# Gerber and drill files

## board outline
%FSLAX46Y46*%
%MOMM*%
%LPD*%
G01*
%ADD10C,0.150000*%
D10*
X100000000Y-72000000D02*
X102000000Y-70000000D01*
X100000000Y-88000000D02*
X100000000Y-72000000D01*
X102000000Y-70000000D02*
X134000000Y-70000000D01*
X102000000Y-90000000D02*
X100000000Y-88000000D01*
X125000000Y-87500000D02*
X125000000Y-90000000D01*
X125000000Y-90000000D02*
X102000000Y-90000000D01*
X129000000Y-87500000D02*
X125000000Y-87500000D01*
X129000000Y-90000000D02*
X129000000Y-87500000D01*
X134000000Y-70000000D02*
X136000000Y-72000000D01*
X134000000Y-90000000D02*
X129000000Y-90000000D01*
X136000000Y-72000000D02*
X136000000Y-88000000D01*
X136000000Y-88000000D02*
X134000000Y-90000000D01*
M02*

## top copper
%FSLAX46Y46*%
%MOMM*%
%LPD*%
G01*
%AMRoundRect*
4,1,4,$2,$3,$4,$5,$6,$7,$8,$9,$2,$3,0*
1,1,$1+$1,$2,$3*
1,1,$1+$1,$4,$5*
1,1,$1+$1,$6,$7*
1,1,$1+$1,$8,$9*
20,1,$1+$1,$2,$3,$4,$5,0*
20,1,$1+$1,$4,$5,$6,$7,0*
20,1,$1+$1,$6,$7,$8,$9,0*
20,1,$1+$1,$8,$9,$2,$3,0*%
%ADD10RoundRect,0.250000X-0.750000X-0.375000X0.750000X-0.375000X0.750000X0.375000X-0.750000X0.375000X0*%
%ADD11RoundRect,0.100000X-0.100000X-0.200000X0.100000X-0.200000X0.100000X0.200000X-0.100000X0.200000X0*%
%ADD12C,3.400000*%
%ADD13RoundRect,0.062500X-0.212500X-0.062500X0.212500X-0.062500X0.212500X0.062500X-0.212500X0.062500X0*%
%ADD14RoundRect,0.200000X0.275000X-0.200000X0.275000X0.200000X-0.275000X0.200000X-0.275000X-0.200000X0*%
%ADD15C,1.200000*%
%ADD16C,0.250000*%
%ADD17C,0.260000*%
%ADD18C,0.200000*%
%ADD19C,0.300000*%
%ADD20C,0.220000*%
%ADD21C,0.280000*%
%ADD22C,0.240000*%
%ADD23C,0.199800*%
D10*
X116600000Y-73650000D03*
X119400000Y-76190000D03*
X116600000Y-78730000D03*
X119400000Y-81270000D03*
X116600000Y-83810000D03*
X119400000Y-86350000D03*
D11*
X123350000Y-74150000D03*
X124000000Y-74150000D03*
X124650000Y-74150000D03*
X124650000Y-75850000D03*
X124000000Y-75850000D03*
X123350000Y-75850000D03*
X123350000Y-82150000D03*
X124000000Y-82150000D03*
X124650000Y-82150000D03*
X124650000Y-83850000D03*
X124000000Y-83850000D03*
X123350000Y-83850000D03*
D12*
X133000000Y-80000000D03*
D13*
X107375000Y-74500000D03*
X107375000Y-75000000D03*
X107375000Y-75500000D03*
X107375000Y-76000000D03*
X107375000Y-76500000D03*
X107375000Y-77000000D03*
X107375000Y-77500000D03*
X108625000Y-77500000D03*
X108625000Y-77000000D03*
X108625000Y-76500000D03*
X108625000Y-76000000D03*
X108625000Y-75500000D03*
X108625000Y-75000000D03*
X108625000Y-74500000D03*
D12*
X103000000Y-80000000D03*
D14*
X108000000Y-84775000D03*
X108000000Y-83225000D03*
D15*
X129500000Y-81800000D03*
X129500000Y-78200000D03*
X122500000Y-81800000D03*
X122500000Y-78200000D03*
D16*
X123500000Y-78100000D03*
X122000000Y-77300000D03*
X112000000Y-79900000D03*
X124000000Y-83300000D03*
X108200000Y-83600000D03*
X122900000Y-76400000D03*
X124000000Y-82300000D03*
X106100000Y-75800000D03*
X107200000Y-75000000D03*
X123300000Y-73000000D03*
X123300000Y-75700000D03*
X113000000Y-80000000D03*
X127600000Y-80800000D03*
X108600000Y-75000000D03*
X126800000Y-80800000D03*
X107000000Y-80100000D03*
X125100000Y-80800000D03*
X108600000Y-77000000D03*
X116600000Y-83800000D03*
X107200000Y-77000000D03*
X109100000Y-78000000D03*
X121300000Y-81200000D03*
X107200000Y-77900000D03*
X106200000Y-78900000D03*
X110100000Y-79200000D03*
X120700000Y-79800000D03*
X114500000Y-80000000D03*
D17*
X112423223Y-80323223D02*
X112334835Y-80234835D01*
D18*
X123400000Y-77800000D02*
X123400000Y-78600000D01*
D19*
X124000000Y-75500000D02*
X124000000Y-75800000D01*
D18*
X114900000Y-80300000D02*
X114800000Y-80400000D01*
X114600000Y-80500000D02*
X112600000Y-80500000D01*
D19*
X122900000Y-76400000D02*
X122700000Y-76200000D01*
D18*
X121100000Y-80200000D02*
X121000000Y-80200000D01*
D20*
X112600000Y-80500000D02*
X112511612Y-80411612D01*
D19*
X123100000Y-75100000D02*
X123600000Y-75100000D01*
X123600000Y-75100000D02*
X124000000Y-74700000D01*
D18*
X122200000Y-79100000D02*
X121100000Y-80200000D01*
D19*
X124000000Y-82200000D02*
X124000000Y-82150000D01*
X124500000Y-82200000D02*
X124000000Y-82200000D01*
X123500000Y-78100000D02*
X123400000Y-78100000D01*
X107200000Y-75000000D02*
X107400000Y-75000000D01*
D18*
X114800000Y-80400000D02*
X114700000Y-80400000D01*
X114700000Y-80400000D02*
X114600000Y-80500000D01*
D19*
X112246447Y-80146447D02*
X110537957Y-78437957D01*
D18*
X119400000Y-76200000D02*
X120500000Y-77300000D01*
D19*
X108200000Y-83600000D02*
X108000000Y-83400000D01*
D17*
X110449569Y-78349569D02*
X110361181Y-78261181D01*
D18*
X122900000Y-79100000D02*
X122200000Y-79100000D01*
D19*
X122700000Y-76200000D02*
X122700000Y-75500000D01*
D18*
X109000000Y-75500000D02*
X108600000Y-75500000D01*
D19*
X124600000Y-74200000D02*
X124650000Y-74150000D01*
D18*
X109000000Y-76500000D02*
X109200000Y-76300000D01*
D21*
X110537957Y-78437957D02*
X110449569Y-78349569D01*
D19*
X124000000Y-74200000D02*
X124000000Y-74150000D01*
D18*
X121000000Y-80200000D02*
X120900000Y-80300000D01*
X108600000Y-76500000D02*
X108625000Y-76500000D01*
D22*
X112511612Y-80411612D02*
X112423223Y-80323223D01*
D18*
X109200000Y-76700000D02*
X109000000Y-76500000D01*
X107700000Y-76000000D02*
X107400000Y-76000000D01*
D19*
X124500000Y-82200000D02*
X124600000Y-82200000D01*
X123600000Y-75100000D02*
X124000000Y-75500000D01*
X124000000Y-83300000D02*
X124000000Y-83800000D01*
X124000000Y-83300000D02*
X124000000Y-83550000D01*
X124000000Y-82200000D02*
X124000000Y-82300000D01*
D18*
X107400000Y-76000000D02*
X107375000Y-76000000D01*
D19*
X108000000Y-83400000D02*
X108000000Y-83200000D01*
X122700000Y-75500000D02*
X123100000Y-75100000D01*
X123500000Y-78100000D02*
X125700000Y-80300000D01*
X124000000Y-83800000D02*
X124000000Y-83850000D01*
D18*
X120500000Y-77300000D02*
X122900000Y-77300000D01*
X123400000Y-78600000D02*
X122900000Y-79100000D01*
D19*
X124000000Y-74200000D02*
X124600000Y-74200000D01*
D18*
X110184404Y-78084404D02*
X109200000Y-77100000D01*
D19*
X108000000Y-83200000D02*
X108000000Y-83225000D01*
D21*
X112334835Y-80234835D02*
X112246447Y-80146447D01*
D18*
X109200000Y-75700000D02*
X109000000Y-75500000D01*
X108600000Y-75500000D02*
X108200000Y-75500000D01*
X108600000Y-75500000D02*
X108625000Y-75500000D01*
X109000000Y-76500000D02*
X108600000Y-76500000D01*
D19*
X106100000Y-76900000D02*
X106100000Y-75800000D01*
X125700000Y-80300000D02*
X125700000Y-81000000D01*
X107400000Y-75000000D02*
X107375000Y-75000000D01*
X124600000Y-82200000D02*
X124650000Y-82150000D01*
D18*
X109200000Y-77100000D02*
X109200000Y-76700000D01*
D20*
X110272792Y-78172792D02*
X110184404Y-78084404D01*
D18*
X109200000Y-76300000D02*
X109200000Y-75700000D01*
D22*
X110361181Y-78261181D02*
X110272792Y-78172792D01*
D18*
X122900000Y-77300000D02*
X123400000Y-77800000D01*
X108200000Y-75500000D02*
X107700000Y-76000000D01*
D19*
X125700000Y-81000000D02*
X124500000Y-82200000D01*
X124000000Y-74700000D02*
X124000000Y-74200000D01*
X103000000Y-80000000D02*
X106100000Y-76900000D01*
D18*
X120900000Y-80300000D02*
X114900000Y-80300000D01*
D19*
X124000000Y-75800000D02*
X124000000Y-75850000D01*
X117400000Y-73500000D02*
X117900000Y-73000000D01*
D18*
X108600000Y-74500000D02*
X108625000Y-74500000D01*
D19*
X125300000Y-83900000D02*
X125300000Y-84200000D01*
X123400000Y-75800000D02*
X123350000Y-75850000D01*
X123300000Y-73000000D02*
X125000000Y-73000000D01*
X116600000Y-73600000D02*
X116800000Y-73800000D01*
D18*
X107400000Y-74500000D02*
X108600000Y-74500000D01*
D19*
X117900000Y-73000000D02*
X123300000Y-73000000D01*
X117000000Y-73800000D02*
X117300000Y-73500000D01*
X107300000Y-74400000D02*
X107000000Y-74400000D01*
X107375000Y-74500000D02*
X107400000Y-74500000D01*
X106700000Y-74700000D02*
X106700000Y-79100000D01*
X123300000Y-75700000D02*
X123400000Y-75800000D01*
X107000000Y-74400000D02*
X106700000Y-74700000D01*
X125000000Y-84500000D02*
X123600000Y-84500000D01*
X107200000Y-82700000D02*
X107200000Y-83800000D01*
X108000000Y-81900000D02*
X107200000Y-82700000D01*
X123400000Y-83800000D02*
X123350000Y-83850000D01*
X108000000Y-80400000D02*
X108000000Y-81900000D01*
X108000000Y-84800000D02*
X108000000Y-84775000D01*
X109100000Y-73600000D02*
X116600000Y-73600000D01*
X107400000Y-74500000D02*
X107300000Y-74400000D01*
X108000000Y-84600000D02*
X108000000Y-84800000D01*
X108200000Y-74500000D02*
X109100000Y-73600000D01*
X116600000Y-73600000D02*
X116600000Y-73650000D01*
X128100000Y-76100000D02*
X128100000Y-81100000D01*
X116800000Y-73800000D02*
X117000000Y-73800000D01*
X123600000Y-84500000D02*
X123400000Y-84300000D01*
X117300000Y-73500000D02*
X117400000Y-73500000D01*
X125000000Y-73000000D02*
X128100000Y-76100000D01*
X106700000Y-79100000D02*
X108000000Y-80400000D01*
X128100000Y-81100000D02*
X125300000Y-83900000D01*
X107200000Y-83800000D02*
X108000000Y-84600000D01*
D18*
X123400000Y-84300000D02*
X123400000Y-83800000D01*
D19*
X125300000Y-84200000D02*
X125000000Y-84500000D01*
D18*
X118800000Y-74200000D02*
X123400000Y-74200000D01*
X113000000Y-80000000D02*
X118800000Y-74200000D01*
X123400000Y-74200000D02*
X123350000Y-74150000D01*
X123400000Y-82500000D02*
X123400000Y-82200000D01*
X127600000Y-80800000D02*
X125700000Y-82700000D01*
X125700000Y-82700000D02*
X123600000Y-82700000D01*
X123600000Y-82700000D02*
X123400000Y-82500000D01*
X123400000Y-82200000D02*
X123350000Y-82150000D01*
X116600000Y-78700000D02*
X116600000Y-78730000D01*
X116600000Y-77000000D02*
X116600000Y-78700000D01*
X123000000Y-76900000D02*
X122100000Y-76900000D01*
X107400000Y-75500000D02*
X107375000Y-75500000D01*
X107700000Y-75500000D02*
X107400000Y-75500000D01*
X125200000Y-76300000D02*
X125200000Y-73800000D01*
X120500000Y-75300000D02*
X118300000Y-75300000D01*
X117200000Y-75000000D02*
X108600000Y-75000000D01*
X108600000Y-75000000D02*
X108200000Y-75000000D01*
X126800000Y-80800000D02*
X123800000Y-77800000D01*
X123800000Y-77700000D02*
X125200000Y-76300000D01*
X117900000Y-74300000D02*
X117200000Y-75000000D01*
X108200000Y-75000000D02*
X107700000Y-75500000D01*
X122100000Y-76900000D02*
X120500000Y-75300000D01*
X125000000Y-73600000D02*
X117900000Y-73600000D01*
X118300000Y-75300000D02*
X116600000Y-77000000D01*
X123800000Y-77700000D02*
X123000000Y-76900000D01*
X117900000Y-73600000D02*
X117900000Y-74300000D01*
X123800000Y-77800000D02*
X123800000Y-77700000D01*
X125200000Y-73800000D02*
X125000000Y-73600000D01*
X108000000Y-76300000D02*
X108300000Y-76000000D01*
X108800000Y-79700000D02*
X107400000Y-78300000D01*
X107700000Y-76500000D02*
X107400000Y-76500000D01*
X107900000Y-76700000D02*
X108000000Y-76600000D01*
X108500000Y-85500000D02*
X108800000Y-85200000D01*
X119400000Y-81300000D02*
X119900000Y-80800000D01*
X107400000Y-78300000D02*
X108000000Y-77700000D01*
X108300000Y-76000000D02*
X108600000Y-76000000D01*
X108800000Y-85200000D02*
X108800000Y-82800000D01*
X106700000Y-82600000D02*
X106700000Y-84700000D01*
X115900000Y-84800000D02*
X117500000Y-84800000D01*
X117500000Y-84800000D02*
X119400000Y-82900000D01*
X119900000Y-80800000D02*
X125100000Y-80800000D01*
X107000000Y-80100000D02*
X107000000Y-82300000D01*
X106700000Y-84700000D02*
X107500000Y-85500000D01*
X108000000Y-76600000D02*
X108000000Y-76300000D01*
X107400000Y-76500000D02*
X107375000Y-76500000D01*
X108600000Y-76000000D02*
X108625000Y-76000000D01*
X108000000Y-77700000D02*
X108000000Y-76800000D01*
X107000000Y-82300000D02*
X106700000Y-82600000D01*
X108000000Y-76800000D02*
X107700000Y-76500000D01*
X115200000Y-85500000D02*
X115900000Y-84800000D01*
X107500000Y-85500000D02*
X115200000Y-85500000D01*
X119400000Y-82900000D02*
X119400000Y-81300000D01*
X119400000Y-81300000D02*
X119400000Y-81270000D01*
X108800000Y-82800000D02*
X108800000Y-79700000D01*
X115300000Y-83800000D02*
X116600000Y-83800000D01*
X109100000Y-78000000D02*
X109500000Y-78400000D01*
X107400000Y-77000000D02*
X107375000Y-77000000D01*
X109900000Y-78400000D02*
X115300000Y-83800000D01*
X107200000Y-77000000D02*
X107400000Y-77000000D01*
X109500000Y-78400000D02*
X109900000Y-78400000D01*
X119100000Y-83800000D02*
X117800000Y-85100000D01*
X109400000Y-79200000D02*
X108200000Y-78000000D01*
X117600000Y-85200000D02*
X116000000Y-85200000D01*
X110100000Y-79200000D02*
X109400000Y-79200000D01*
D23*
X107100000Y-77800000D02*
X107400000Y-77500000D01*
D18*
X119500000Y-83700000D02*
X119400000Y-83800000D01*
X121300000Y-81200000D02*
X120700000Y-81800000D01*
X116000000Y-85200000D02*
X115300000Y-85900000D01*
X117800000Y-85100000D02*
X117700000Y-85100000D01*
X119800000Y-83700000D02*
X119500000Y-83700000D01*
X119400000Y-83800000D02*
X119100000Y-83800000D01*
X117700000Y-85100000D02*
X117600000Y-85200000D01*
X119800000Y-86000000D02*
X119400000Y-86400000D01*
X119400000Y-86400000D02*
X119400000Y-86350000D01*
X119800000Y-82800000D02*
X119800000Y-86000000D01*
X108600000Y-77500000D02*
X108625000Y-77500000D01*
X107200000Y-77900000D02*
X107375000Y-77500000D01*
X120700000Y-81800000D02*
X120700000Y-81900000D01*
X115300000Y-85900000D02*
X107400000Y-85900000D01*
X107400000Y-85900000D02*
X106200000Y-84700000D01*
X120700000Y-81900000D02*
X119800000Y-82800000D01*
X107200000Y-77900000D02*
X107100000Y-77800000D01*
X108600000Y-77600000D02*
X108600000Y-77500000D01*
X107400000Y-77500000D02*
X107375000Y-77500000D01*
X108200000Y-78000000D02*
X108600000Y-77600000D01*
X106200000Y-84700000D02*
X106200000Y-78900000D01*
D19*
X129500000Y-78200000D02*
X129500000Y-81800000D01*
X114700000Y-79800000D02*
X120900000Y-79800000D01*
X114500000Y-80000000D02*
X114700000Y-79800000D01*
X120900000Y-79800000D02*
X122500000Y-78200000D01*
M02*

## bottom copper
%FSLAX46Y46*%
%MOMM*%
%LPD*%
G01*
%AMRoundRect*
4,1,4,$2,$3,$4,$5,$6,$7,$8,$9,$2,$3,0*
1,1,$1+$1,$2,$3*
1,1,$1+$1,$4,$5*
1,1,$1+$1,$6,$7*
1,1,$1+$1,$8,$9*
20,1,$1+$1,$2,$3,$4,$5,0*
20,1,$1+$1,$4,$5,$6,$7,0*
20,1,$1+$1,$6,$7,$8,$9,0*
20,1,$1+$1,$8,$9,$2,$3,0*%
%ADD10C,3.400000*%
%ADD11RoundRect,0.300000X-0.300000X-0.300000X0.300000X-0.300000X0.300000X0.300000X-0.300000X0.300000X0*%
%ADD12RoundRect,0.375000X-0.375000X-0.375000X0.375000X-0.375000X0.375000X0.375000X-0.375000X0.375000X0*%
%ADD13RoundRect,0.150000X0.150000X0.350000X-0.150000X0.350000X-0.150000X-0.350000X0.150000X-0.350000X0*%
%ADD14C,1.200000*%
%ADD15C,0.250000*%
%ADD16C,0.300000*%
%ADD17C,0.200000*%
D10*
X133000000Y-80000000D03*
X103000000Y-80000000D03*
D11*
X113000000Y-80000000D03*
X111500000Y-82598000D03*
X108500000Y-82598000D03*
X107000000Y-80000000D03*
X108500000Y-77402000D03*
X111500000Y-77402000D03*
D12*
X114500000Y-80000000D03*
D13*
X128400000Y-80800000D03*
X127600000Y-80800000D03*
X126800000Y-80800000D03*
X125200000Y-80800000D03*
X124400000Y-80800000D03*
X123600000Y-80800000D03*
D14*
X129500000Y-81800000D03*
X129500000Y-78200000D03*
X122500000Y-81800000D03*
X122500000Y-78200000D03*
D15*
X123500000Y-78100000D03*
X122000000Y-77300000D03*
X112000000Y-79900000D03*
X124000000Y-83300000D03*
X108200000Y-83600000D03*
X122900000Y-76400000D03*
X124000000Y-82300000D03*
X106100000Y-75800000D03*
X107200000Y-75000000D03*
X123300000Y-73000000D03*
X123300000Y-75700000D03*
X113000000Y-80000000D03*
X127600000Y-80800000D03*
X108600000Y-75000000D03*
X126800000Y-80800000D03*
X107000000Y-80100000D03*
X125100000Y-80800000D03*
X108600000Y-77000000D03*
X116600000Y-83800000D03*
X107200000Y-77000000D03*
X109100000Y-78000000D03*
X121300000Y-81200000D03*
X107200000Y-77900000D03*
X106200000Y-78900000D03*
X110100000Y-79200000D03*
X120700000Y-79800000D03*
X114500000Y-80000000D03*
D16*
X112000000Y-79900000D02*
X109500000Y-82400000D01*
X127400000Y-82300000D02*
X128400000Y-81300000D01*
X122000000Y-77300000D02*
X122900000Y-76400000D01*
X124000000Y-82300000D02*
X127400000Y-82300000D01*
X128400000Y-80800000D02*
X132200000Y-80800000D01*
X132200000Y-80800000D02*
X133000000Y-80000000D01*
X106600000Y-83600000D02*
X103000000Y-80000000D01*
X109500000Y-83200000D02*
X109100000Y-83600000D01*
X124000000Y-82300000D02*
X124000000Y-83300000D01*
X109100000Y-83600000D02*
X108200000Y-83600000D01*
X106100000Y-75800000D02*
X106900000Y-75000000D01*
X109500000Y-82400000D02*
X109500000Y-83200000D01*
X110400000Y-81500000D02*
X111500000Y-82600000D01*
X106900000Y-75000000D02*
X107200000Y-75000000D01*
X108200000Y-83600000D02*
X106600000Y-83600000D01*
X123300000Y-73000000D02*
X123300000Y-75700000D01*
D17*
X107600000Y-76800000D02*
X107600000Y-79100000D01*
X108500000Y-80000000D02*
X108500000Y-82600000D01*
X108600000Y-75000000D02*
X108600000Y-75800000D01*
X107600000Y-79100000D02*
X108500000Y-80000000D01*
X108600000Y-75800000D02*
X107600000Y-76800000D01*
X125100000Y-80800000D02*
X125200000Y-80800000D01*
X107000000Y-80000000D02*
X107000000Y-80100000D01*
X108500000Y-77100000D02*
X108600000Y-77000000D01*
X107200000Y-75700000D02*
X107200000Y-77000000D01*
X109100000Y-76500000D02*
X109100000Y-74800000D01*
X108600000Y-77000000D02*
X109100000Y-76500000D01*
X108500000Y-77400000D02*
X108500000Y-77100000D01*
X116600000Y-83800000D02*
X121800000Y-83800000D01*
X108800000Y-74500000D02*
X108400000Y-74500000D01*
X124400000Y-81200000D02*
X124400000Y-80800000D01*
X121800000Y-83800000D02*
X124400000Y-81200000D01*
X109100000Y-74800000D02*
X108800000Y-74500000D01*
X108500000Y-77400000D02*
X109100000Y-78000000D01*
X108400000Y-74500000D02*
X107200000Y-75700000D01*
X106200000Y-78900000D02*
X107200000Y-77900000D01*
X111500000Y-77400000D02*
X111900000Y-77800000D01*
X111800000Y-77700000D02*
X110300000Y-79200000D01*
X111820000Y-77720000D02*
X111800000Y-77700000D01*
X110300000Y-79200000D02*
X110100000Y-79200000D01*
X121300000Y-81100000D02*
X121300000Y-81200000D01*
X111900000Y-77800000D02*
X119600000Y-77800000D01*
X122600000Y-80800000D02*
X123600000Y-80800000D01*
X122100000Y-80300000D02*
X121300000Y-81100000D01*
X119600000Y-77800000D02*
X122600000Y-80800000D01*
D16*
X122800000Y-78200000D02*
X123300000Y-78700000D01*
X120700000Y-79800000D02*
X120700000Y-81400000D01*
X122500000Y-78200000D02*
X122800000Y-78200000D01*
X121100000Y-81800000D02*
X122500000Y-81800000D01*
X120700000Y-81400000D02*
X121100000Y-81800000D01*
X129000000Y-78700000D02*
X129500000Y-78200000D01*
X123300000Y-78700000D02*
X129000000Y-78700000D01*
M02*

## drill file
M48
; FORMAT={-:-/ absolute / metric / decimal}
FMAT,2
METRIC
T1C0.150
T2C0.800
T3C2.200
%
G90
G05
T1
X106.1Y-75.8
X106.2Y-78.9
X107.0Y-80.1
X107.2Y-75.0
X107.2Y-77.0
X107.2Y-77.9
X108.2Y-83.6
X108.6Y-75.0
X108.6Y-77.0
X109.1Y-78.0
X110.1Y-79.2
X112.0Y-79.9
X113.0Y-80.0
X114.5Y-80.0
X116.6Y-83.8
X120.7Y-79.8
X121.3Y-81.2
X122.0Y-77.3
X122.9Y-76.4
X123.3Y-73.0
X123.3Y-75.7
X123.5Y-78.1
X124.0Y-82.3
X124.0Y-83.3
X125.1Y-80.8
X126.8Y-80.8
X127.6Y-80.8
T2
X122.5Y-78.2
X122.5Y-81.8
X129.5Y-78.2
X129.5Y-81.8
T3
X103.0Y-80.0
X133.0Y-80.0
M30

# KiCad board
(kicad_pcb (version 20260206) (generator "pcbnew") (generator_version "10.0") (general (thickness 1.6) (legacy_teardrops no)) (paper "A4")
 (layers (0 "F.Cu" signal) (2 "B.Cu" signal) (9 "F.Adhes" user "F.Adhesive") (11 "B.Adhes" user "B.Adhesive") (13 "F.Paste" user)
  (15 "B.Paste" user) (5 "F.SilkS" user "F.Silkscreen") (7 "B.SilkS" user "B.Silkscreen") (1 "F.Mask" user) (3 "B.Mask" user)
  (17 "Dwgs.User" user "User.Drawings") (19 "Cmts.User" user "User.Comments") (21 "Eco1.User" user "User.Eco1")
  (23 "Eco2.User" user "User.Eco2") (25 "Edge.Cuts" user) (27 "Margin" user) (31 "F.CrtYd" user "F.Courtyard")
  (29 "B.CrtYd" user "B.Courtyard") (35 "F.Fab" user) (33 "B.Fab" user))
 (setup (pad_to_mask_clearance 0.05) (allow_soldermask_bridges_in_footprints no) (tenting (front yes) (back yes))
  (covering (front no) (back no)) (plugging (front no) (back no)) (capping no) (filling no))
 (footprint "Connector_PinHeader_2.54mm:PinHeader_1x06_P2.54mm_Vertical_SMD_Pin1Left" (layer "F.Cu") (at 118 73.65)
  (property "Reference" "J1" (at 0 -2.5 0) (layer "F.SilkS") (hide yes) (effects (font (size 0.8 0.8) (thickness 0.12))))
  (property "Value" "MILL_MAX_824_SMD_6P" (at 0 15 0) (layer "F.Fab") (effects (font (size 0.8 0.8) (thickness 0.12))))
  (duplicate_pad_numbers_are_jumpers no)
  (pad "1" smd roundrect (at -1.4 0) (size 2 1.25) (layers "F.Cu" "F.Mask" "F.Paste") (roundrect_rratio 0.2) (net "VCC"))
  (pad "2" smd roundrect (at 1.4 2.54) (size 2 1.25) (layers "F.Cu" "F.Mask" "F.Paste") (roundrect_rratio 0.2) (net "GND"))
  (pad "3" smd roundrect (at -1.4 5.08) (size 2 1.25) (layers "F.Cu" "F.Mask" "F.Paste") (roundrect_rratio 0.2) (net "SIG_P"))
  (pad "4" smd roundrect (at 1.4 7.62) (size 2 1.25) (layers "F.Cu" "F.Mask" "F.Paste") (roundrect_rratio 0.2) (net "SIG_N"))
  (pad "5" smd roundrect (at -1.4 10.16) (size 2 1.25) (layers "F.Cu" "F.Mask" "F.Paste") (roundrect_rratio 0.2) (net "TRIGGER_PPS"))
  (pad "6" smd roundrect (at 1.4 12.7) (size 2 1.25) (layers "F.Cu" "F.Mask" "F.Paste") (roundrect_rratio 0.2) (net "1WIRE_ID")))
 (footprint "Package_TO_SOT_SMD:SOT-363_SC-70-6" (layer "F.Cu") (at 124 75)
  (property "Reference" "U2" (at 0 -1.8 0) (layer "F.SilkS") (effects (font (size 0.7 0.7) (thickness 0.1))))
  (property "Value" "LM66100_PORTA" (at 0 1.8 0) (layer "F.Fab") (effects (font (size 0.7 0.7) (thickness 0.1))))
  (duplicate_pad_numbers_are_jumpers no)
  (pad "1" smd roundrect (at -0.65 -0.85) (size 0.4 0.6) (layers "F.Cu" "F.Mask" "F.Paste") (roundrect_rratio 0.25) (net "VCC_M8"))
  (pad "2" smd roundrect (at 0 -0.85) (size 0.4 0.6) (layers "F.Cu" "F.Mask" "F.Paste") (roundrect_rratio 0.25) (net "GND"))
  (pad "3" smd roundrect (at 0.65 -0.85) (size 0.4 0.6) (layers "F.Cu" "F.Mask" "F.Paste") (roundrect_rratio 0.25) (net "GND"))
  (pad "4" smd roundrect (at 0.65 0.85) (size 0.4 0.6) (layers "F.Cu" "F.Mask" "F.Paste") (roundrect_rratio 0.25))
  (pad "5" smd roundrect (at 0 0.85) (size 0.4 0.6) (layers "F.Cu" "F.Mask" "F.Paste") (roundrect_rratio 0.25) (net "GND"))
  (pad "6" smd roundrect (at -0.65 0.85) (size 0.4 0.6) (layers "F.Cu" "F.Mask" "F.Paste") (roundrect_rratio 0.25) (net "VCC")))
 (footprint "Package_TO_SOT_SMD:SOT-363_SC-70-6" (layer "F.Cu") (at 124 83)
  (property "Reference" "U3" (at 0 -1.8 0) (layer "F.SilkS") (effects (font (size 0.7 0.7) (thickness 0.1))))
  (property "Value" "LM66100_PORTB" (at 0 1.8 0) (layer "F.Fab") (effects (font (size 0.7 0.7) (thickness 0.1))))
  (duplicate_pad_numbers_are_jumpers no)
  (pad "1" smd roundrect (at -0.65 -0.85) (size 0.4 0.6) (layers "F.Cu" "F.Mask" "F.Paste") (roundrect_rratio 0.25) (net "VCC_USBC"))
  (pad "2" smd roundrect (at 0 -0.85) (size 0.4 0.6) (layers "F.Cu" "F.Mask" "F.Paste") (roundrect_rratio 0.25) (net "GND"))
  (pad "3" smd roundrect (at 0.65 -0.85) (size 0.4 0.6) (layers "F.Cu" "F.Mask" "F.Paste") (roundrect_rratio 0.25) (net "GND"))
  (pad "4" smd roundrect (at 0.65 0.85) (size 0.4 0.6) (layers "F.Cu" "F.Mask" "F.Paste") (roundrect_rratio 0.25))
  (pad "5" smd roundrect (at 0 0.85) (size 0.4 0.6) (layers "F.Cu" "F.Mask" "F.Paste") (roundrect_rratio 0.25) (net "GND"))
  (pad "6" smd roundrect (at -0.65 0.85) (size 0.4 0.6) (layers "F.Cu" "F.Mask" "F.Paste") (roundrect_rratio 0.25) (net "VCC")))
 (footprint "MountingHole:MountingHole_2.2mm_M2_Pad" (layer "F.Cu") (at 133 80)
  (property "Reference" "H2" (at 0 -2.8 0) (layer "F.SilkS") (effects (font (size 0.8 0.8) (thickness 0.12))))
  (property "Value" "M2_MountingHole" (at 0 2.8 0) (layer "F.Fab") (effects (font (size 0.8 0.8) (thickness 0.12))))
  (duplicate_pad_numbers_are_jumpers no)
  (pad "1" thru_hole circle (at 0 0) (size 3.4 3.4) (drill 2.2) (layers "*.Cu" "*.Mask") (remove_unused_layers no) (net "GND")))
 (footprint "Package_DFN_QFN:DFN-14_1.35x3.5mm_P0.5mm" (layer "F.Cu") (at 108 76)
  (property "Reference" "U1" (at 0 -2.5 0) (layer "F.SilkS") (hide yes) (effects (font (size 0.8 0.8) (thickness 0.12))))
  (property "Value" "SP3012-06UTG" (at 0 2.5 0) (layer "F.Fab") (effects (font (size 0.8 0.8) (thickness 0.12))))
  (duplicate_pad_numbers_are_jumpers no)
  (pad "1" smd roundrect (at -0.625 -1.5) (size 0.55 0.25) (layers "F.Cu" "F.Mask" "F.Paste") (roundrect_rratio 0.25) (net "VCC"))
  (pad "2" smd roundrect (at -0.625 -1) (size 0.55 0.25) (layers "F.Cu" "F.Mask" "F.Paste") (roundrect_rratio 0.25) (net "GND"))
  (pad "3" smd roundrect (at -0.625 -0.5) (size 0.55 0.25) (layers "F.Cu" "F.Mask" "F.Paste") (roundrect_rratio 0.25) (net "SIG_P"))
  (pad "4" smd roundrect (at -0.625 0) (size 0.55 0.25) (layers "F.Cu" "F.Mask" "F.Paste") (roundrect_rratio 0.25) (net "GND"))
  (pad "5" smd roundrect (at -0.625 0.5) (size 0.55 0.25) (layers "F.Cu" "F.Mask" "F.Paste") (roundrect_rratio 0.25) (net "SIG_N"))
  (pad "6" smd roundrect (at -0.625 1) (size 0.55 0.25) (layers "F.Cu" "F.Mask" "F.Paste") (roundrect_rratio 0.25) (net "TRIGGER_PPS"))
  (pad "7" smd roundrect (at -0.625 1.5) (size 0.55 0.25) (layers "F.Cu" "F.Mask" "F.Paste") (roundrect_rratio 0.25) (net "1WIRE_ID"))
  (pad "8" smd roundrect (at 0.625 1.5) (size 0.55 0.25) (layers "F.Cu" "F.Mask" "F.Paste") (roundrect_rratio 0.25) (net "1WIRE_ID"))
  (pad "9" smd roundrect (at 0.625 1) (size 0.55 0.25) (layers "F.Cu" "F.Mask" "F.Paste") (roundrect_rratio 0.25) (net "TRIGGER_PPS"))
  (pad "10" smd roundrect (at 0.625 0.5) (size 0.55 0.25) (layers "F.Cu" "F.Mask" "F.Paste") (roundrect_rratio 0.25) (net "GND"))
  (pad "11" smd roundrect (at 0.625 0) (size 0.55 0.25) (layers "F.Cu" "F.Mask" "F.Paste") (roundrect_rratio 0.25) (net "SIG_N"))
  (pad "12" smd roundrect (at 0.625 -0.5) (size 0.55 0.25) (layers "F.Cu" "F.Mask" "F.Paste") (roundrect_rratio 0.25) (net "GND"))
  (pad "13" smd roundrect (at 0.625 -1) (size 0.55 0.25) (layers "F.Cu" "F.Mask" "F.Paste") (roundrect_rratio 0.25) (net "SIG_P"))
  (pad "14" smd roundrect (at 0.625 -1.5) (size 0.55 0.25) (layers "F.Cu" "F.Mask" "F.Paste") (roundrect_rratio 0.25) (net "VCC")))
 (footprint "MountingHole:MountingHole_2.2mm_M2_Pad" (layer "F.Cu") (at 103 80)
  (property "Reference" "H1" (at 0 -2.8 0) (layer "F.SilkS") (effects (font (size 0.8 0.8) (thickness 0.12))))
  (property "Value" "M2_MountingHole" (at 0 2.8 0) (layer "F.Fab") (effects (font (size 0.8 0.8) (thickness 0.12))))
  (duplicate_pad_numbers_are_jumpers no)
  (pad "1" thru_hole circle (at 0 0) (size 3.4 3.4) (drill 2.2) (layers "*.Cu" "*.Mask") (remove_unused_layers no) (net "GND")))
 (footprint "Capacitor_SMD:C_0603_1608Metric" (layer "F.Cu") (at 108 84 90)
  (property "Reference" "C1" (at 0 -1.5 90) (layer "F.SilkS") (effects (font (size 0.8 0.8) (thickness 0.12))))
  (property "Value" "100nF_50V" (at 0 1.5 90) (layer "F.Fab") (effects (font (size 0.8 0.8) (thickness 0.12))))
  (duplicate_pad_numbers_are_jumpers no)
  (pad "1" smd roundrect (at -0.775 0 90) (size 0.8 0.95) (layers "F.Cu" "F.Mask" "F.Paste") (roundrect_rratio 0.25) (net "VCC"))
  (pad "2" smd roundrect (at 0.775 0 90) (size 0.8 0.95) (layers "F.Cu" "F.Mask" "F.Paste") (roundrect_rratio 0.25) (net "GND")))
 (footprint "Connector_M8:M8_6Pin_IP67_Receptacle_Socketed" (layer "B.Cu") (at 110 80)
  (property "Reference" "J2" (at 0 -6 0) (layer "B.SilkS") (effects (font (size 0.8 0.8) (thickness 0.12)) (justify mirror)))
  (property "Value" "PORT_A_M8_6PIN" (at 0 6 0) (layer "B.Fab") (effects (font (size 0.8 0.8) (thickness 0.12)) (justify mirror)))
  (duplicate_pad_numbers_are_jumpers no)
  (pad "1" smd roundrect (at 3 0) (size 1.2 1.2) (layers "B.Cu" "B.Mask" "B.Paste") (roundrect_rratio 0.25) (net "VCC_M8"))
  (pad "2" smd roundrect (at 1.5 2.598) (size 1.2 1.2) (layers "B.Cu" "B.Mask" "B.Paste") (roundrect_rratio 0.25) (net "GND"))
  (pad "3" smd roundrect (at -1.5 2.598) (size 1.2 1.2) (layers "B.Cu" "B.Mask" "B.Paste") (roundrect_rratio 0.25) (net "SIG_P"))
  (pad "4" smd roundrect (at -3 0) (size 1.2 1.2) (layers "B.Cu" "B.Mask" "B.Paste") (roundrect_rratio 0.25) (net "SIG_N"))
  (pad "5" smd roundrect (at -1.5 -2.598) (size 1.2 1.2) (layers "B.Cu" "B.Mask" "B.Paste") (roundrect_rratio 0.25) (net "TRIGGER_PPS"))
  (pad "6" smd roundrect (at 1.5 -2.598) (size 1.2 1.2) (layers "B.Cu" "B.Mask" "B.Paste") (roundrect_rratio 0.25) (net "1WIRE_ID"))
  (pad "7" smd roundrect (at 4.5 0) (size 1.5 1.5) (layers "B.Cu" "B.Mask" "B.Paste") (roundrect_rratio 0.25) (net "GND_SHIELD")))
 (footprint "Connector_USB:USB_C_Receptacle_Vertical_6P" (layer "B.Cu") (at 126 80 180)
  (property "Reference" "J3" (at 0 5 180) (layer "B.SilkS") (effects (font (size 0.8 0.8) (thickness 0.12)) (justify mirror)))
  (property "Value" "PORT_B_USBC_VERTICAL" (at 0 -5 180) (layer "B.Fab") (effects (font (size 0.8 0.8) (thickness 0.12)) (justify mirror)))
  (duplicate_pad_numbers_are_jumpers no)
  (pad "1" smd roundrect (at -2.4 -0.8 180) (size 0.6 1) (layers "B.Cu" "B.Mask" "B.Paste") (roundrect_rratio 0.25) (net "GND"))
  (pad "2" smd roundrect (at -1.6 -0.8 180) (size 0.6 1) (layers "B.Cu" "B.Mask" "B.Paste") (roundrect_rratio 0.25) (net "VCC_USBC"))
  (pad "3" smd roundrect (at -0.8 -0.8 180) (size 0.6 1) (layers "B.Cu" "B.Mask" "B.Paste") (roundrect_rratio 0.25) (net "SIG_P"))
  (pad "4" smd roundrect (at 0.8 -0.8 180) (size 0.6 1) (layers "B.Cu" "B.Mask" "B.Paste") (roundrect_rratio 0.25) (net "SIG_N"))
  (pad "5" smd roundrect (at 1.6 -0.8 180) (size 0.6 1) (layers "B.Cu" "B.Mask" "B.Paste") (roundrect_rratio 0.25) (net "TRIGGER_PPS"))
  (pad "6" smd roundrect (at 2.4 -0.8 180) (size 0.6 1) (layers "B.Cu" "B.Mask" "B.Paste") (roundrect_rratio 0.25) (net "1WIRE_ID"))
  (pad "SH" thru_hole circle (at -3.5 -1.8 180) (size 1.2 1.2) (drill 0.8) (layers "*.Cu" "*.Mask" "B.Paste") (remove_unused_layers no)
   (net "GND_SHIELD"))
  (pad "SH" thru_hole circle (at -3.5 1.8 180) (size 1.2 1.2) (drill 0.8) (layers "*.Cu" "*.Mask" "B.Paste") (remove_unused_layers no)
   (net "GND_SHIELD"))
  (pad "SH" thru_hole circle (at 3.5 -1.8 180) (size 1.2 1.2) (drill 0.8) (layers "*.Cu" "*.Mask" "B.Paste") (remove_unused_layers no)
   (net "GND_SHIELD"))
  (pad "SH" thru_hole circle (at 3.5 1.8 180) (size 1.2 1.2) (drill 0.8) (layers "*.Cu" "*.Mask" "B.Paste") (remove_unused_layers no)
   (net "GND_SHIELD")))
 (gr_line (start 100 72) (end 102 70) (stroke (width 0.15) (type solid)) (layer "Edge.Cuts"))
 (gr_line (start 100 88) (end 100 72) (stroke (width 0.15) (type solid)) (layer "Edge.Cuts"))
 (gr_line (start 102 70) (end 134 70) (stroke (width 0.15) (type solid)) (layer "Edge.Cuts"))
 (gr_line (start 102 90) (end 100 88) (stroke (width 0.15) (type solid)) (layer "Edge.Cuts"))
 (gr_line (start 125 87.5) (end 125 90) (stroke (width 0.15) (type solid)) (layer "Edge.Cuts"))
 (gr_line (start 125 90) (end 102 90) (stroke (width 0.15) (type solid)) (layer "Edge.Cuts"))
 (gr_line (start 129 87.5) (end 125 87.5) (stroke (width 0.15) (type solid)) (layer "Edge.Cuts"))
 (gr_line (start 129 90) (end 129 87.5) (stroke (width 0.15) (type solid)) (layer "Edge.Cuts"))
 (gr_line (start 134 70) (end 136 72) (stroke (width 0.15) (type solid)) (layer "Edge.Cuts"))
 (gr_line (start 134 90) (end 129 90) (stroke (width 0.15) (type solid)) (layer "Edge.Cuts"))
 (gr_line (start 136 72) (end 136 88) (stroke (width 0.15) (type solid)) (layer "Edge.Cuts"))
 (gr_line (start 136 88) (end 134 90) (stroke (width 0.15) (type solid)) (layer "Edge.Cuts"))
 (segment (start 112.423223 80.323223) (end 112.334835 80.234835) (width 0.26) (layer "F.Cu") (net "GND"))
 (segment (start 123.4 77.8) (end 123.4 78.6) (width 0.2) (layer "F.Cu") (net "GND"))
 (segment (start 124 75.5) (end 124 75.8) (width 0.3) (layer "F.Cu") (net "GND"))
 (segment (start 114.9 80.3) (end 114.8 80.4) (width 0.2) (layer "F.Cu") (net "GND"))
 (segment (start 114.6 80.5) (end 112.6 80.5) (width 0.2) (layer "F.Cu") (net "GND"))
 (segment (start 122.9 76.4) (end 122.7 76.2) (width 0.3) (layer "F.Cu") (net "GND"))
 (segment (start 121.1 80.2) (end 121 80.2) (width 0.2) (layer "F.Cu") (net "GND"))
 (segment (start 112.6 80.5) (end 112.511612 80.411612) (width 0.22) (layer "F.Cu") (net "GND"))
 (segment (start 123.1 75.1) (end 123.6 75.1) (width 0.3) (layer "F.Cu") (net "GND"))
 (segment (start 123.6 75.1) (end 124 74.7) (width 0.3) (layer "F.Cu") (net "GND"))
 (segment (start 122.2 79.1) (end 121.1 80.2) (width 0.2) (layer "F.Cu") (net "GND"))
 (segment (start 124 82.2) (end 124 82.15) (width 0.3) (layer "F.Cu") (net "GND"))
 (segment (start 124.5 82.2) (end 124 82.2) (width 0.3) (layer "F.Cu") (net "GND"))
 (segment (start 123.5 78.1) (end 123.4 78.1) (width 0.3) (layer "F.Cu") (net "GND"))
 (segment (start 107.2 75) (end 107.4 75) (width 0.3) (layer "F.Cu") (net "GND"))
 (segment (start 114.8 80.4) (end 114.7 80.4) (width 0.2) (layer "F.Cu") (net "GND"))
 (segment (start 114.7 80.4) (end 114.6 80.5) (width 0.2) (layer "F.Cu") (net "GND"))
 (segment (start 112.246447 80.146447) (end 110.537957 78.437957) (width 0.3) (layer "F.Cu") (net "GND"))
 (segment (start 119.4 76.2) (end 120.5 77.3) (width 0.2) (layer "F.Cu") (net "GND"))
 (segment (start 108.2 83.6) (end 108 83.4) (width 0.3) (layer "F.Cu") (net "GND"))
 (segment (start 110.449569 78.349569) (end 110.361181 78.261181) (width 0.26) (layer "F.Cu") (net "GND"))
 (segment (start 122.9 79.1) (end 122.2 79.1) (width 0.2) (layer "F.Cu") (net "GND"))
 (segment (start 122.7 76.2) (end 122.7 75.5) (width 0.3) (layer "F.Cu") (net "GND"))
 (segment (start 109 75.5) (end 108.6 75.5) (width 0.2) (layer "F.Cu") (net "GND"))
 (segment (start 124.6 74.2) (end 124.65 74.15) (width 0.3) (layer "F.Cu") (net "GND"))
 (segment (start 109 76.5) (end 109.2 76.3) (width 0.2) (layer "F.Cu") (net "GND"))
 (segment (start 110.537957 78.437957) (end 110.449569 78.349569) (width 0.28) (layer "F.Cu") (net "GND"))
 (segment (start 124 74.2) (end 124 74.15) (width 0.3) (layer "F.Cu") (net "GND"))
 (segment (start 121 80.2) (end 120.9 80.3) (width 0.2) (layer "F.Cu") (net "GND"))
 (segment (start 108.6 76.5) (end 108.625 76.5) (width 0.2) (layer "F.Cu") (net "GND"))
 (segment (start 112.511612 80.411612) (end 112.423223 80.323223) (width 0.24) (layer "F.Cu") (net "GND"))
 (segment (start 109.2 76.7) (end 109 76.5) (width 0.2) (layer "F.Cu") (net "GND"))
 (segment (start 107.7 76) (end 107.4 76) (width 0.2) (layer "F.Cu") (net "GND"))
 (segment (start 124.5 82.2) (end 124.6 82.2) (width 0.3) (layer "F.Cu") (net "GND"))
 (segment (start 123.6 75.1) (end 124 75.5) (width 0.3) (layer "F.Cu") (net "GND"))
 (segment (start 124 83.3) (end 124 83.8) (width 0.3) (layer "F.Cu") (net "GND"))
 (segment (start 124 83.3) (end 124 83.55) (width 0.3) (layer "F.Cu") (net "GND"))
 (segment (start 124 82.2) (end 124 82.3) (width 0.3) (layer "F.Cu") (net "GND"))
 (segment (start 107.4 76) (end 107.375 76) (width 0.2) (layer "F.Cu") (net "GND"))
 (segment (start 108 83.4) (end 108 83.2) (width 0.3) (layer "F.Cu") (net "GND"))
 (segment (start 122.7 75.5) (end 123.1 75.1) (width 0.3) (layer "F.Cu") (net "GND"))
 (segment (start 123.5 78.1) (end 125.7 80.3) (width 0.3) (layer "F.Cu") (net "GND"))
 (segment (start 124 83.8) (end 124 83.85) (width 0.3) (layer "F.Cu") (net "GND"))
 (segment (start 120.5 77.3) (end 122.9 77.3) (width 0.2) (layer "F.Cu") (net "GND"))
 (segment (start 123.4 78.6) (end 122.9 79.1) (width 0.2) (layer "F.Cu") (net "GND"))
 (segment (start 124 74.2) (end 124.6 74.2) (width 0.3) (layer "F.Cu") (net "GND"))
 (segment (start 110.184404 78.084404) (end 109.2 77.1) (width 0.2) (layer "F.Cu") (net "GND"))
 (segment (start 108 83.2) (end 108 83.225) (width 0.3) (layer "F.Cu") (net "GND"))
 (segment (start 112.334835 80.234835) (end 112.246447 80.146447) (width 0.28) (layer "F.Cu") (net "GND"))
 (segment (start 109.2 75.7) (end 109 75.5) (width 0.2) (layer "F.Cu") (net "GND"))
 (segment (start 108.6 75.5) (end 108.2 75.5) (width 0.2) (layer "F.Cu") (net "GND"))
 (segment (start 108.6 75.5) (end 108.625 75.5) (width 0.2) (layer "F.Cu") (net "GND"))
 (segment (start 109 76.5) (end 108.6 76.5) (width 0.2) (layer "F.Cu") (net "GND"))
 (segment (start 106.1 76.9) (end 106.1 75.8) (width 0.3) (layer "F.Cu") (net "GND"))
 (segment (start 125.7 80.3) (end 125.7 81) (width 0.3) (layer "F.Cu") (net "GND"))
 (segment (start 107.4 75) (end 107.375 75) (width 0.3) (layer "F.Cu") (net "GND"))
 (segment (start 124.6 82.2) (end 124.65 82.15) (width 0.3) (layer "F.Cu") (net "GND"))
 (segment (start 109.2 77.1) (end 109.2 76.7) (width 0.2) (layer "F.Cu") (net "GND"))
 (segment (start 110.272792 78.172792) (end 110.184404 78.084404) (width 0.22) (layer "F.Cu") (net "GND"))
 (segment (start 109.2 76.3) (end 109.2 75.7) (width 0.2) (layer "F.Cu") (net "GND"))
 (segment (start 110.361181 78.261181) (end 110.272792 78.172792) (width 0.24) (layer "F.Cu") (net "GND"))
 (segment (start 122.9 77.3) (end 123.4 77.8) (width 0.2) (layer "F.Cu") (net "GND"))
 (segment (start 108.2 75.5) (end 107.7 76) (width 0.2) (layer "F.Cu") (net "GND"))
 (segment (start 125.7 81) (end 124.5 82.2) (width 0.3) (layer "F.Cu") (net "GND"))
 (segment (start 124 74.7) (end 124 74.2) (width 0.3) (layer "F.Cu") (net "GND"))
 (segment (start 103 80) (end 106.1 76.9) (width 0.3) (layer "F.Cu") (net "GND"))
 (segment (start 120.9 80.3) (end 114.9 80.3) (width 0.2) (layer "F.Cu") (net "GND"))
 (segment (start 124 75.8) (end 124 75.85) (width 0.3) (layer "F.Cu") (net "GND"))
 (via (at 123.5 78.1) (size 0.25) (drill 0.15) (layers "F.Cu" "B.Cu") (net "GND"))
 (via (at 122 77.3) (size 0.25) (drill 0.15) (layers "F.Cu" "B.Cu") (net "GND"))
 (via (at 112 79.9) (size 0.25) (drill 0.15) (layers "F.Cu" "B.Cu") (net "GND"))
 (via (at 124 83.3) (size 0.25) (drill 0.15) (layers "F.Cu" "B.Cu") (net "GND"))
 (via (at 108.2 83.6) (size 0.25) (drill 0.15) (layers "F.Cu" "B.Cu") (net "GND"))
 (via (at 122.9 76.4) (size 0.25) (drill 0.15) (layers "F.Cu" "B.Cu") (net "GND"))
 (via (at 124 82.3) (size 0.25) (drill 0.15) (layers "F.Cu" "B.Cu") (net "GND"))
 (via (at 106.1 75.8) (size 0.25) (drill 0.15) (layers "F.Cu" "B.Cu") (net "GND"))
 (via (at 107.2 75) (size 0.25) (drill 0.15) (layers "F.Cu" "B.Cu") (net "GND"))
 (segment (start 112 79.9) (end 109.5 82.4) (width 0.3) (layer "B.Cu") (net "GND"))
 (segment (start 127.4 82.3) (end 128.4 81.3) (width 0.3) (layer "B.Cu") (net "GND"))
 (segment (start 122 77.3) (end 122.9 76.4) (width 0.3) (layer "B.Cu") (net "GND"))
 (segment (start 124 82.3) (end 127.4 82.3) (width 0.3) (layer "B.Cu") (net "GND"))
 (segment (start 128.4 80.8) (end 132.2 80.8) (width 0.3) (layer "B.Cu") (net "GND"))
 (segment (start 132.2 80.8) (end 133 80) (width 0.3) (layer "B.Cu") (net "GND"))
 (segment (start 106.6 83.6) (end 103 80) (width 0.3) (layer "B.Cu") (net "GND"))
 (segment (start 109.5 83.2) (end 109.1 83.6) (width 0.3) (layer "B.Cu") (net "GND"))
 (segment (start 124 82.3) (end 124 83.3) (width 0.3) (layer "B.Cu") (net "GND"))
 (segment (start 109.1 83.6) (end 108.2 83.6) (width 0.3) (layer "B.Cu") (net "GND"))
 (segment (start 106.1 75.8) (end 106.9 75) (width 0.3) (layer "B.Cu") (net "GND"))
 (segment (start 109.5 82.4) (end 109.5 83.2) (width 0.3) (layer "B.Cu") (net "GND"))
 (segment (start 110.4 81.5) (end 111.5 82.6) (width 0.3) (layer "B.Cu") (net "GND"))
 (segment (start 106.9 75) (end 107.2 75) (width 0.3) (layer "B.Cu") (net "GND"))
 (segment (start 108.2 83.6) (end 106.6 83.6) (width 0.3) (layer "B.Cu") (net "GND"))
 (segment (start 117.4 73.5) (end 117.9 73) (width 0.3) (layer "F.Cu") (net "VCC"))
 (segment (start 108.6 74.5) (end 108.625 74.5) (width 0.2) (layer "F.Cu") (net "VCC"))
 (segment (start 125.3 83.9) (end 125.3 84.2) (width 0.3) (layer "F.Cu") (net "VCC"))
 (segment (start 123.4 75.8) (end 123.35 75.85) (width 0.3) (layer "F.Cu") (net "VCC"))
 (segment (start 123.3 73) (end 125 73) (width 0.3) (layer "F.Cu") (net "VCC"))
 (segment (start 116.6 73.6) (end 116.8 73.8) (width 0.3) (layer "F.Cu") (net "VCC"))
 (segment (start 107.4 74.5) (end 108.6 74.5) (width 0.2) (layer "F.Cu") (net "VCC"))
 (segment (start 117.9 73) (end 123.3 73) (width 0.3) (layer "F.Cu") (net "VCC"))
 (segment (start 117 73.8) (end 117.3 73.5) (width 0.3) (layer "F.Cu") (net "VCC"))
 (segment (start 107.3 74.4) (end 107 74.4) (width 0.3) (layer "F.Cu") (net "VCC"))
 (segment (start 107.375 74.5) (end 107.4 74.5) (width 0.3) (layer "F.Cu") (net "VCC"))
 (segment (start 106.7 74.7) (end 106.7 79.1) (width 0.3) (layer "F.Cu") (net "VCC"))
 (segment (start 123.3 75.7) (end 123.4 75.8) (width 0.3) (layer "F.Cu") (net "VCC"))
 (segment (start 107 74.4) (end 106.7 74.7) (width 0.3) (layer "F.Cu") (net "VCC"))
 (segment (start 125 84.5) (end 123.6 84.5) (width 0.3) (layer "F.Cu") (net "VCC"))
 (segment (start 107.2 82.7) (end 107.2 83.8) (width 0.3) (layer "F.Cu") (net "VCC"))
 (segment (start 108 81.9) (end 107.2 82.7) (width 0.3) (layer "F.Cu") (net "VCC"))
 (segment (start 123.4 83.8) (end 123.35 83.85) (width 0.3) (layer "F.Cu") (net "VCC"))
 (segment (start 108 80.4) (end 108 81.9) (width 0.3) (layer "F.Cu") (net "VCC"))
 (segment (start 108 84.8) (end 108 84.775) (width 0.3) (layer "F.Cu") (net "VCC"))
 (segment (start 109.1 73.6) (end 116.6 73.6) (width 0.3) (layer "F.Cu") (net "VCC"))
 (segment (start 107.4 74.5) (end 107.3 74.4) (width 0.3) (layer "F.Cu") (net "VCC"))
 (segment (start 108 84.6) (end 108 84.8) (width 0.3) (layer "F.Cu") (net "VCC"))
 (segment (start 108.2 74.5) (end 109.1 73.6) (width 0.3) (layer "F.Cu") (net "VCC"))
 (segment (start 116.6 73.6) (end 116.6 73.65) (width 0.3) (layer "F.Cu") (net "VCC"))
 (segment (start 128.1 76.1) (end 128.1 81.1) (width 0.3) (layer "F.Cu") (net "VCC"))
 (segment (start 116.8 73.8) (end 117 73.8) (width 0.3) (layer "F.Cu") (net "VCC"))
 (segment (start 123.6 84.5) (end 123.4 84.3) (width 0.3) (layer "F.Cu") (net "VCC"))
 (segment (start 117.3 73.5) (end 117.4 73.5) (width 0.3) (layer "F.Cu") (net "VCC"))
 (segment (start 125 73) (end 128.1 76.1) (width 0.3) (layer "F.Cu") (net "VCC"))
 (segment (start 106.7 79.1) (end 108 80.4) (width 0.3) (layer "F.Cu") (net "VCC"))
 (segment (start 128.1 81.1) (end 125.3 83.9) (width 0.3) (layer "F.Cu") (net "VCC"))
 (segment (start 107.2 83.8) (end 108 84.6) (width 0.3) (layer "F.Cu") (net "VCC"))
 (segment (start 123.4 84.3) (end 123.4 83.8) (width 0.2) (layer "F.Cu") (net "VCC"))
 (segment (start 125.3 84.2) (end 125 84.5) (width 0.3) (layer "F.Cu") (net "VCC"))
 (via (at 123.3 73) (size 0.25) (drill 0.15) (layers "F.Cu" "B.Cu") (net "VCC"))
 (via (at 123.3 75.7) (size 0.25) (drill 0.15) (layers "F.Cu" "B.Cu") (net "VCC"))
 (segment (start 123.3 73) (end 123.3 75.7) (width 0.3) (layer "B.Cu") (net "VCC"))
 (segment (start 118.8 74.2) (end 123.4 74.2) (width 0.2) (layer "F.Cu") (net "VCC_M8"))
 (segment (start 113 80) (end 118.8 74.2) (width 0.2) (layer "F.Cu") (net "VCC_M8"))
 (segment (start 123.4 74.2) (end 123.35 74.15) (width 0.2) (layer "F.Cu") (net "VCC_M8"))
 (via (at 113 80) (size 0.25) (drill 0.15) (layers "F.Cu" "B.Cu") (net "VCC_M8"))
 (segment (start 123.4 82.5) (end 123.4 82.2) (width 0.2) (layer "F.Cu") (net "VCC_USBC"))
 (segment (start 127.6 80.8) (end 125.7 82.7) (width 0.2) (layer "F.Cu") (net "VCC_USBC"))
 (segment (start 125.7 82.7) (end 123.6 82.7) (width 0.2) (layer "F.Cu") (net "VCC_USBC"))
 (segment (start 123.6 82.7) (end 123.4 82.5) (width 0.2) (layer "F.Cu") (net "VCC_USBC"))
 (segment (start 123.4 82.2) (end 123.35 82.15) (width 0.2) (layer "F.Cu") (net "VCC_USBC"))
 (via (at 127.6 80.8) (size 0.25) (drill 0.15) (layers "F.Cu" "B.Cu") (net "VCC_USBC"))
 (segment (start 116.6 78.7) (end 116.6 78.73) (width 0.2) (layer "F.Cu") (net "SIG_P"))
 (segment (start 116.6 77) (end 116.6 78.7) (width 0.2) (layer "F.Cu") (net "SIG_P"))
 (segment (start 123 76.9) (end 122.1 76.9) (width 0.2) (layer "F.Cu") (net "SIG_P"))
 (segment (start 107.4 75.5) (end 107.375 75.5) (width 0.2) (layer "F.Cu") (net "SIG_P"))
 (segment (start 107.7 75.5) (end 107.4 75.5) (width 0.2) (layer "F.Cu") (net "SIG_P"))
 (segment (start 125.2 76.3) (end 125.2 73.8) (width 0.2) (layer "F.Cu") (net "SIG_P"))
 (segment (start 120.5 75.3) (end 118.3 75.3) (width 0.2) (layer "F.Cu") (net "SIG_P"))
 (segment (start 117.2 75) (end 108.6 75) (width 0.2) (layer "F.Cu") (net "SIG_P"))
 (segment (start 108.6 75) (end 108.2 75) (width 0.2) (layer "F.Cu") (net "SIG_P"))
 (segment (start 126.8 80.8) (end 123.8 77.8) (width 0.2) (layer "F.Cu") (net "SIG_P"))
 (segment (start 123.8 77.7) (end 125.2 76.3) (width 0.2) (layer "F.Cu") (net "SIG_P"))
 (segment (start 117.9 74.3) (end 117.2 75) (width 0.2) (layer "F.Cu") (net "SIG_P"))
 (segment (start 108.2 75) (end 107.7 75.5) (width 0.2) (layer "F.Cu") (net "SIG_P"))
 (segment (start 122.1 76.9) (end 120.5 75.3) (width 0.2) (layer "F.Cu") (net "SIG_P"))
 (segment (start 125 73.6) (end 117.9 73.6) (width 0.2) (layer "F.Cu") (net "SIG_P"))
 (segment (start 118.3 75.3) (end 116.6 77) (width 0.2) (layer "F.Cu") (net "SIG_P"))
 (segment (start 123.8 77.7) (end 123 76.9) (width 0.2) (layer "F.Cu") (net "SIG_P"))
 (segment (start 117.9 73.6) (end 117.9 74.3) (width 0.2) (layer "F.Cu") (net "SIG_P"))
 (segment (start 123.8 77.8) (end 123.8 77.7) (width 0.2) (layer "F.Cu") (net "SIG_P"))
 (segment (start 125.2 73.8) (end 125 73.6) (width 0.2) (layer "F.Cu") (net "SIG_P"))
 (via (at 108.6 75) (size 0.25) (drill 0.15) (layers "F.Cu" "B.Cu") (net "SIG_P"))
 (via (at 126.8 80.8) (size 0.25) (drill 0.15) (layers "F.Cu" "B.Cu") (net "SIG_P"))
 (segment (start 107.6 76.8) (end 107.6 79.1) (width 0.2) (layer "B.Cu") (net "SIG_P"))
 (segment (start 108.5 80) (end 108.5 82.6) (width 0.2) (layer "B.Cu") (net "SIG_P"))
 (segment (start 108.6 75) (end 108.6 75.8) (width 0.2) (layer "B.Cu") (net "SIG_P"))
 (segment (start 107.6 79.1) (end 108.5 80) (width 0.2) (layer "B.Cu") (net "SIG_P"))
 (segment (start 108.6 75.8) (end 107.6 76.8) (width 0.2) (layer "B.Cu") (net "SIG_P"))
 (segment (start 108 76.3) (end 108.3 76) (width 0.2) (layer "F.Cu") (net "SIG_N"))
 (segment (start 108.8 79.7) (end 107.4 78.3) (width 0.2) (layer "F.Cu") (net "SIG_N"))
 (segment (start 107.7 76.5) (end 107.4 76.5) (width 0.2) (layer "F.Cu") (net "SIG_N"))
 (segment (start 107.9 76.7) (end 108 76.6) (width 0.2) (layer "F.Cu") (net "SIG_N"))
 (segment (start 108.5 85.5) (end 108.8 85.2) (width 0.2) (layer "F.Cu") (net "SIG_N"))
 (segment (start 119.4 81.3) (end 119.9 80.8) (width 0.2) (layer "F.Cu") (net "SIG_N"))
 (segment (start 107.4 78.3) (end 108 77.7) (width 0.2) (layer "F.Cu") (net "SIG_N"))
 (segment (start 108.3 76) (end 108.6 76) (width 0.2) (layer "F.Cu") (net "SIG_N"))
 (segment (start 108.8 85.2) (end 108.8 82.8) (width 0.2) (layer "F.Cu") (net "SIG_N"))
 (segment (start 106.7 82.6) (end 106.7 84.7) (width 0.2) (layer "F.Cu") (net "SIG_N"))
 (segment (start 115.9 84.8) (end 117.5 84.8) (width 0.2) (layer "F.Cu") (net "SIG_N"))
 (segment (start 117.5 84.8) (end 119.4 82.9) (width 0.2) (layer "F.Cu") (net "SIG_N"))
 (segment (start 119.9 80.8) (end 125.1 80.8) (width 0.2) (layer "F.Cu") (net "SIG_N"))
 (segment (start 107 80.1) (end 107 82.3) (width 0.2) (layer "F.Cu") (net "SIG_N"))
 (segment (start 106.7 84.7) (end 107.5 85.5) (width 0.2) (layer "F.Cu") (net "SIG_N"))
 (segment (start 108 76.6) (end 108 76.3) (width 0.2) (layer "F.Cu") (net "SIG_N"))
 (segment (start 107.4 76.5) (end 107.375 76.5) (width 0.2) (layer "F.Cu") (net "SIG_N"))
 (segment (start 108.6 76) (end 108.625 76) (width 0.2) (layer "F.Cu") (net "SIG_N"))
 (segment (start 108 77.7) (end 108 76.8) (width 0.2) (layer "F.Cu") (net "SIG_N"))
 (segment (start 107 82.3) (end 106.7 82.6) (width 0.2) (layer "F.Cu") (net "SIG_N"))
 (segment (start 108 76.8) (end 107.7 76.5) (width 0.2) (layer "F.Cu") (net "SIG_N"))
 (segment (start 115.2 85.5) (end 115.9 84.8) (width 0.2) (layer "F.Cu") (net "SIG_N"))
 (segment (start 107.5 85.5) (end 115.2 85.5) (width 0.2) (layer "F.Cu") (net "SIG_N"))
 (segment (start 119.4 82.9) (end 119.4 81.3) (width 0.2) (layer "F.Cu") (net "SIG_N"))
 (segment (start 119.4 81.3) (end 119.4 81.27) (width 0.2) (layer "F.Cu") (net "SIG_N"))
 (segment (start 108.8 82.8) (end 108.8 79.7) (width 0.2) (layer "F.Cu") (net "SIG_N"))
 (via (at 107 80.1) (size 0.25) (drill 0.15) (layers "F.Cu" "B.Cu") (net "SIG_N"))
 (via (at 125.1 80.8) (size 0.25) (drill 0.15) (layers "F.Cu" "B.Cu") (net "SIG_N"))
 (segment (start 125.1 80.8) (end 125.2 80.8) (width 0.2) (layer "B.Cu") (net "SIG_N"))
 (segment (start 107 80) (end 107 80.1) (width 0.2) (layer "B.Cu") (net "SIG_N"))
 (segment (start 115.3 83.8) (end 116.6 83.8) (width 0.2) (layer "F.Cu") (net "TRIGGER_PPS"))
 (segment (start 109.1 78) (end 109.5 78.4) (width 0.2) (layer "F.Cu") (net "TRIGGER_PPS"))
 (segment (start 107.4 77) (end 107.375 77) (width 0.2) (layer "F.Cu") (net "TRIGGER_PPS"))
 (segment (start 109.9 78.4) (end 115.3 83.8) (width 0.2) (layer "F.Cu") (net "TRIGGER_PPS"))
 (segment (start 107.2 77) (end 107.4 77) (width 0.2) (layer "F.Cu") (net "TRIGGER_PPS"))
 (segment (start 109.5 78.4) (end 109.9 78.4) (width 0.2) (layer "F.Cu") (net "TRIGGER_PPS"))
 (via (at 108.6 77) (size 0.25) (drill 0.15) (layers "F.Cu" "B.Cu") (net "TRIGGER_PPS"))
 (via (at 116.6 83.8) (size 0.25) (drill 0.15) (layers "F.Cu" "B.Cu") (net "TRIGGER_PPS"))
 (via (at 107.2 77) (size 0.25) (drill 0.15) (layers "F.Cu" "B.Cu") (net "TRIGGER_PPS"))
 (via (at 109.1 78) (size 0.25) (drill 0.15) (layers "F.Cu" "B.Cu") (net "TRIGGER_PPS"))
 (segment (start 108.5 77.1) (end 108.6 77) (width 0.2) (layer "B.Cu") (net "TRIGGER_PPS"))
 (segment (start 107.2 75.7) (end 107.2 77) (width 0.2) (layer "B.Cu") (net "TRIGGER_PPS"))
 (segment (start 109.1 76.5) (end 109.1 74.8) (width 0.2) (layer "B.Cu") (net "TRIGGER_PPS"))
 (segment (start 108.6 77) (end 109.1 76.5) (width 0.2) (layer "B.Cu") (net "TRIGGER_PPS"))
 (segment (start 108.5 77.4) (end 108.5 77.1) (width 0.2) (layer "B.Cu") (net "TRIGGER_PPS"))
 (segment (start 116.6 83.8) (end 121.8 83.8) (width 0.2) (layer "B.Cu") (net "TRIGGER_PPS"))
 (segment (start 108.8 74.5) (end 108.4 74.5) (width 0.2) (layer "B.Cu") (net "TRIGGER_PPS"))
 (segment (start 124.4 81.2) (end 124.4 80.8) (width 0.2) (layer "B.Cu") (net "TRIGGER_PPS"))
 (segment (start 121.8 83.8) (end 124.4 81.2) (width 0.2) (layer "B.Cu") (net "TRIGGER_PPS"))
 (segment (start 109.1 74.8) (end 108.8 74.5) (width 0.2) (layer "B.Cu") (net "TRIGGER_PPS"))
 (segment (start 108.5 77.4) (end 109.1 78) (width 0.2) (layer "B.Cu") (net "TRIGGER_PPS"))
 (segment (start 108.4 74.5) (end 107.2 75.7) (width 0.2) (layer "B.Cu") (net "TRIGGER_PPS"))
 (segment (start 119.1 83.8) (end 117.8 85.1) (width 0.2) (layer "F.Cu") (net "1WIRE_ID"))
 (segment (start 109.4 79.2) (end 108.2 78) (width 0.2) (layer "F.Cu") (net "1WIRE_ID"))
 (segment (start 117.6 85.2) (end 116 85.2) (width 0.2) (layer "F.Cu") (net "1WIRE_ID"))
 (segment (start 110.1 79.2) (end 109.4 79.2) (width 0.2) (layer "F.Cu") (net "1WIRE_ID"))
 (segment (start 107.1 77.8) (end 107.4 77.5) (width 0.1998) (layer "F.Cu") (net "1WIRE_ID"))
 (segment (start 119.5 83.7) (end 119.4 83.8) (width 0.2) (layer "F.Cu") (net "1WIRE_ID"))
 (segment (start 121.3 81.2) (end 120.7 81.8) (width 0.2) (layer "F.Cu") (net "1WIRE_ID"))
 (segment (start 116 85.2) (end 115.3 85.9) (width 0.2) (layer "F.Cu") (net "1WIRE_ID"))
 (segment (start 117.8 85.1) (end 117.7 85.1) (width 0.2) (layer "F.Cu") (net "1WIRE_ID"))
 (segment (start 119.8 83.7) (end 119.5 83.7) (width 0.2) (layer "F.Cu") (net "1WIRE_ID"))
 (segment (start 119.4 83.8) (end 119.1 83.8) (width 0.2) (layer "F.Cu") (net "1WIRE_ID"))
 (segment (start 117.7 85.1) (end 117.6 85.2) (width 0.2) (layer "F.Cu") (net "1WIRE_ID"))
 (segment (start 119.8 86) (end 119.4 86.4) (width 0.2) (layer "F.Cu") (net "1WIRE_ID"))
 (segment (start 119.4 86.4) (end 119.4 86.35) (width 0.2) (layer "F.Cu") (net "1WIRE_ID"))
 (segment (start 119.8 82.8) (end 119.8 86) (width 0.2) (layer "F.Cu") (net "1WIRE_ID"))
 (segment (start 108.6 77.5) (end 108.625 77.5) (width 0.2) (layer "F.Cu") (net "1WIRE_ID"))
 (segment (start 107.2 77.9) (end 107.375 77.5) (width 0.2) (layer "F.Cu") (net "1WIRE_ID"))
 (segment (start 120.7 81.8) (end 120.7 81.9) (width 0.2) (layer "F.Cu") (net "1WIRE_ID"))
 (segment (start 115.3 85.9) (end 107.4 85.9) (width 0.2) (layer "F.Cu") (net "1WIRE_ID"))
 (segment (start 107.4 85.9) (end 106.2 84.7) (width 0.2) (layer "F.Cu") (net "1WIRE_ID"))
 (segment (start 120.7 81.9) (end 119.8 82.8) (width 0.2) (layer "F.Cu") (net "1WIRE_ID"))
 (segment (start 107.2 77.9) (end 107.1 77.8) (width 0.2) (layer "F.Cu") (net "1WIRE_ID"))
 (segment (start 108.6 77.6) (end 108.6 77.5) (width 0.2) (layer "F.Cu") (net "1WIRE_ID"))
 (segment (start 107.4 77.5) (end 107.375 77.5) (width 0.2) (layer "F.Cu") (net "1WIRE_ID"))
 (segment (start 108.2 78) (end 108.6 77.6) (width 0.2) (layer "F.Cu") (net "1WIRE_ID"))
 (segment (start 106.2 84.7) (end 106.2 78.9) (width 0.2) (layer "F.Cu") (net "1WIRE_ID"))
 (via (at 121.3 81.2) (size 0.25) (drill 0.15) (layers "F.Cu" "B.Cu") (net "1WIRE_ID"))
 (via (at 107.2 77.9) (size 0.25) (drill 0.15) (layers "F.Cu" "B.Cu") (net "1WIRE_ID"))
 (via (at 106.2 78.9) (size 0.25) (drill 0.15) (layers "F.Cu" "B.Cu") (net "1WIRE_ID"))
 (via (at 110.1 79.2) (size 0.25) (drill 0.15) (layers "F.Cu" "B.Cu") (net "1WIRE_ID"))
 (segment (start 106.2 78.9) (end 107.2 77.9) (width 0.2) (layer "B.Cu") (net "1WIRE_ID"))
 (segment (start 111.5 77.4) (end 111.9 77.8) (width 0.2) (layer "B.Cu") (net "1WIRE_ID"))
 (segment (start 111.8 77.7) (end 110.3 79.2) (width 0.2) (layer "B.Cu") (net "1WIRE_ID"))
 (segment (start 111.82 77.72) (end 111.8 77.7) (width 0.2) (layer "B.Cu") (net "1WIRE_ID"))
 (segment (start 110.3 79.2) (end 110.1 79.2) (width 0.2) (layer "B.Cu") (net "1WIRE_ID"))
 (segment (start 121.3 81.1) (end 121.3 81.2) (width 0.2) (layer "B.Cu") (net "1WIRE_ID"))
 (segment (start 111.9 77.8) (end 119.6 77.8) (width 0.2) (layer "B.Cu") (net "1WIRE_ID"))
 (segment (start 122.6 80.8) (end 123.6 80.8) (width 0.2) (layer "B.Cu") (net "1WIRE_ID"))
 (segment (start 122.1 80.3) (end 121.3 81.1) (width 0.2) (layer "B.Cu") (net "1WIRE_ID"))
 (segment (start 119.6 77.8) (end 122.6 80.8) (width 0.2) (layer "B.Cu") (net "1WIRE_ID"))
 (segment (start 129.5 78.2) (end 129.5 81.8) (width 0.3) (layer "F.Cu") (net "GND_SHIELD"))
 (segment (start 114.7 79.8) (end 120.9 79.8) (width 0.3) (layer "F.Cu") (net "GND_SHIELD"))
 (segment (start 114.5 80) (end 114.7 79.8) (width 0.3) (layer "F.Cu") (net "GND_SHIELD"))
 (segment (start 120.9 79.8) (end 122.5 78.2) (width 0.3) (layer "F.Cu") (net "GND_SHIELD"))
 (via (at 120.7 79.8) (size 0.25) (drill 0.15) (layers "F.Cu" "B.Cu") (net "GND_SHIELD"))
 (via (at 114.5 80) (size 0.25) (drill 0.15) (layers "F.Cu" "B.Cu") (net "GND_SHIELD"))
 (segment (start 122.8 78.2) (end 123.3 78.7) (width 0.3) (layer "B.Cu") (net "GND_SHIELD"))
 (segment (start 120.7 79.8) (end 120.7 81.4) (width 0.3) (layer "B.Cu") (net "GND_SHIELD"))
 (segment (start 122.5 78.2) (end 122.8 78.2) (width 0.3) (layer "B.Cu") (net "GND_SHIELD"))
 (segment (start 121.1 81.8) (end 122.5 81.8) (width 0.3) (layer "B.Cu") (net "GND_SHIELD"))
 (segment (start 120.7 81.4) (end 121.1 81.8) (width 0.3) (layer "B.Cu") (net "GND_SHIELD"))
 (segment (start 129 78.7) (end 129.5 78.2) (width 0.3) (layer "B.Cu") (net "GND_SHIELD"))
 (segment (start 123.3 78.7) (end 129 78.7) (width 0.3) (layer "B.Cu") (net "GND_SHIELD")))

